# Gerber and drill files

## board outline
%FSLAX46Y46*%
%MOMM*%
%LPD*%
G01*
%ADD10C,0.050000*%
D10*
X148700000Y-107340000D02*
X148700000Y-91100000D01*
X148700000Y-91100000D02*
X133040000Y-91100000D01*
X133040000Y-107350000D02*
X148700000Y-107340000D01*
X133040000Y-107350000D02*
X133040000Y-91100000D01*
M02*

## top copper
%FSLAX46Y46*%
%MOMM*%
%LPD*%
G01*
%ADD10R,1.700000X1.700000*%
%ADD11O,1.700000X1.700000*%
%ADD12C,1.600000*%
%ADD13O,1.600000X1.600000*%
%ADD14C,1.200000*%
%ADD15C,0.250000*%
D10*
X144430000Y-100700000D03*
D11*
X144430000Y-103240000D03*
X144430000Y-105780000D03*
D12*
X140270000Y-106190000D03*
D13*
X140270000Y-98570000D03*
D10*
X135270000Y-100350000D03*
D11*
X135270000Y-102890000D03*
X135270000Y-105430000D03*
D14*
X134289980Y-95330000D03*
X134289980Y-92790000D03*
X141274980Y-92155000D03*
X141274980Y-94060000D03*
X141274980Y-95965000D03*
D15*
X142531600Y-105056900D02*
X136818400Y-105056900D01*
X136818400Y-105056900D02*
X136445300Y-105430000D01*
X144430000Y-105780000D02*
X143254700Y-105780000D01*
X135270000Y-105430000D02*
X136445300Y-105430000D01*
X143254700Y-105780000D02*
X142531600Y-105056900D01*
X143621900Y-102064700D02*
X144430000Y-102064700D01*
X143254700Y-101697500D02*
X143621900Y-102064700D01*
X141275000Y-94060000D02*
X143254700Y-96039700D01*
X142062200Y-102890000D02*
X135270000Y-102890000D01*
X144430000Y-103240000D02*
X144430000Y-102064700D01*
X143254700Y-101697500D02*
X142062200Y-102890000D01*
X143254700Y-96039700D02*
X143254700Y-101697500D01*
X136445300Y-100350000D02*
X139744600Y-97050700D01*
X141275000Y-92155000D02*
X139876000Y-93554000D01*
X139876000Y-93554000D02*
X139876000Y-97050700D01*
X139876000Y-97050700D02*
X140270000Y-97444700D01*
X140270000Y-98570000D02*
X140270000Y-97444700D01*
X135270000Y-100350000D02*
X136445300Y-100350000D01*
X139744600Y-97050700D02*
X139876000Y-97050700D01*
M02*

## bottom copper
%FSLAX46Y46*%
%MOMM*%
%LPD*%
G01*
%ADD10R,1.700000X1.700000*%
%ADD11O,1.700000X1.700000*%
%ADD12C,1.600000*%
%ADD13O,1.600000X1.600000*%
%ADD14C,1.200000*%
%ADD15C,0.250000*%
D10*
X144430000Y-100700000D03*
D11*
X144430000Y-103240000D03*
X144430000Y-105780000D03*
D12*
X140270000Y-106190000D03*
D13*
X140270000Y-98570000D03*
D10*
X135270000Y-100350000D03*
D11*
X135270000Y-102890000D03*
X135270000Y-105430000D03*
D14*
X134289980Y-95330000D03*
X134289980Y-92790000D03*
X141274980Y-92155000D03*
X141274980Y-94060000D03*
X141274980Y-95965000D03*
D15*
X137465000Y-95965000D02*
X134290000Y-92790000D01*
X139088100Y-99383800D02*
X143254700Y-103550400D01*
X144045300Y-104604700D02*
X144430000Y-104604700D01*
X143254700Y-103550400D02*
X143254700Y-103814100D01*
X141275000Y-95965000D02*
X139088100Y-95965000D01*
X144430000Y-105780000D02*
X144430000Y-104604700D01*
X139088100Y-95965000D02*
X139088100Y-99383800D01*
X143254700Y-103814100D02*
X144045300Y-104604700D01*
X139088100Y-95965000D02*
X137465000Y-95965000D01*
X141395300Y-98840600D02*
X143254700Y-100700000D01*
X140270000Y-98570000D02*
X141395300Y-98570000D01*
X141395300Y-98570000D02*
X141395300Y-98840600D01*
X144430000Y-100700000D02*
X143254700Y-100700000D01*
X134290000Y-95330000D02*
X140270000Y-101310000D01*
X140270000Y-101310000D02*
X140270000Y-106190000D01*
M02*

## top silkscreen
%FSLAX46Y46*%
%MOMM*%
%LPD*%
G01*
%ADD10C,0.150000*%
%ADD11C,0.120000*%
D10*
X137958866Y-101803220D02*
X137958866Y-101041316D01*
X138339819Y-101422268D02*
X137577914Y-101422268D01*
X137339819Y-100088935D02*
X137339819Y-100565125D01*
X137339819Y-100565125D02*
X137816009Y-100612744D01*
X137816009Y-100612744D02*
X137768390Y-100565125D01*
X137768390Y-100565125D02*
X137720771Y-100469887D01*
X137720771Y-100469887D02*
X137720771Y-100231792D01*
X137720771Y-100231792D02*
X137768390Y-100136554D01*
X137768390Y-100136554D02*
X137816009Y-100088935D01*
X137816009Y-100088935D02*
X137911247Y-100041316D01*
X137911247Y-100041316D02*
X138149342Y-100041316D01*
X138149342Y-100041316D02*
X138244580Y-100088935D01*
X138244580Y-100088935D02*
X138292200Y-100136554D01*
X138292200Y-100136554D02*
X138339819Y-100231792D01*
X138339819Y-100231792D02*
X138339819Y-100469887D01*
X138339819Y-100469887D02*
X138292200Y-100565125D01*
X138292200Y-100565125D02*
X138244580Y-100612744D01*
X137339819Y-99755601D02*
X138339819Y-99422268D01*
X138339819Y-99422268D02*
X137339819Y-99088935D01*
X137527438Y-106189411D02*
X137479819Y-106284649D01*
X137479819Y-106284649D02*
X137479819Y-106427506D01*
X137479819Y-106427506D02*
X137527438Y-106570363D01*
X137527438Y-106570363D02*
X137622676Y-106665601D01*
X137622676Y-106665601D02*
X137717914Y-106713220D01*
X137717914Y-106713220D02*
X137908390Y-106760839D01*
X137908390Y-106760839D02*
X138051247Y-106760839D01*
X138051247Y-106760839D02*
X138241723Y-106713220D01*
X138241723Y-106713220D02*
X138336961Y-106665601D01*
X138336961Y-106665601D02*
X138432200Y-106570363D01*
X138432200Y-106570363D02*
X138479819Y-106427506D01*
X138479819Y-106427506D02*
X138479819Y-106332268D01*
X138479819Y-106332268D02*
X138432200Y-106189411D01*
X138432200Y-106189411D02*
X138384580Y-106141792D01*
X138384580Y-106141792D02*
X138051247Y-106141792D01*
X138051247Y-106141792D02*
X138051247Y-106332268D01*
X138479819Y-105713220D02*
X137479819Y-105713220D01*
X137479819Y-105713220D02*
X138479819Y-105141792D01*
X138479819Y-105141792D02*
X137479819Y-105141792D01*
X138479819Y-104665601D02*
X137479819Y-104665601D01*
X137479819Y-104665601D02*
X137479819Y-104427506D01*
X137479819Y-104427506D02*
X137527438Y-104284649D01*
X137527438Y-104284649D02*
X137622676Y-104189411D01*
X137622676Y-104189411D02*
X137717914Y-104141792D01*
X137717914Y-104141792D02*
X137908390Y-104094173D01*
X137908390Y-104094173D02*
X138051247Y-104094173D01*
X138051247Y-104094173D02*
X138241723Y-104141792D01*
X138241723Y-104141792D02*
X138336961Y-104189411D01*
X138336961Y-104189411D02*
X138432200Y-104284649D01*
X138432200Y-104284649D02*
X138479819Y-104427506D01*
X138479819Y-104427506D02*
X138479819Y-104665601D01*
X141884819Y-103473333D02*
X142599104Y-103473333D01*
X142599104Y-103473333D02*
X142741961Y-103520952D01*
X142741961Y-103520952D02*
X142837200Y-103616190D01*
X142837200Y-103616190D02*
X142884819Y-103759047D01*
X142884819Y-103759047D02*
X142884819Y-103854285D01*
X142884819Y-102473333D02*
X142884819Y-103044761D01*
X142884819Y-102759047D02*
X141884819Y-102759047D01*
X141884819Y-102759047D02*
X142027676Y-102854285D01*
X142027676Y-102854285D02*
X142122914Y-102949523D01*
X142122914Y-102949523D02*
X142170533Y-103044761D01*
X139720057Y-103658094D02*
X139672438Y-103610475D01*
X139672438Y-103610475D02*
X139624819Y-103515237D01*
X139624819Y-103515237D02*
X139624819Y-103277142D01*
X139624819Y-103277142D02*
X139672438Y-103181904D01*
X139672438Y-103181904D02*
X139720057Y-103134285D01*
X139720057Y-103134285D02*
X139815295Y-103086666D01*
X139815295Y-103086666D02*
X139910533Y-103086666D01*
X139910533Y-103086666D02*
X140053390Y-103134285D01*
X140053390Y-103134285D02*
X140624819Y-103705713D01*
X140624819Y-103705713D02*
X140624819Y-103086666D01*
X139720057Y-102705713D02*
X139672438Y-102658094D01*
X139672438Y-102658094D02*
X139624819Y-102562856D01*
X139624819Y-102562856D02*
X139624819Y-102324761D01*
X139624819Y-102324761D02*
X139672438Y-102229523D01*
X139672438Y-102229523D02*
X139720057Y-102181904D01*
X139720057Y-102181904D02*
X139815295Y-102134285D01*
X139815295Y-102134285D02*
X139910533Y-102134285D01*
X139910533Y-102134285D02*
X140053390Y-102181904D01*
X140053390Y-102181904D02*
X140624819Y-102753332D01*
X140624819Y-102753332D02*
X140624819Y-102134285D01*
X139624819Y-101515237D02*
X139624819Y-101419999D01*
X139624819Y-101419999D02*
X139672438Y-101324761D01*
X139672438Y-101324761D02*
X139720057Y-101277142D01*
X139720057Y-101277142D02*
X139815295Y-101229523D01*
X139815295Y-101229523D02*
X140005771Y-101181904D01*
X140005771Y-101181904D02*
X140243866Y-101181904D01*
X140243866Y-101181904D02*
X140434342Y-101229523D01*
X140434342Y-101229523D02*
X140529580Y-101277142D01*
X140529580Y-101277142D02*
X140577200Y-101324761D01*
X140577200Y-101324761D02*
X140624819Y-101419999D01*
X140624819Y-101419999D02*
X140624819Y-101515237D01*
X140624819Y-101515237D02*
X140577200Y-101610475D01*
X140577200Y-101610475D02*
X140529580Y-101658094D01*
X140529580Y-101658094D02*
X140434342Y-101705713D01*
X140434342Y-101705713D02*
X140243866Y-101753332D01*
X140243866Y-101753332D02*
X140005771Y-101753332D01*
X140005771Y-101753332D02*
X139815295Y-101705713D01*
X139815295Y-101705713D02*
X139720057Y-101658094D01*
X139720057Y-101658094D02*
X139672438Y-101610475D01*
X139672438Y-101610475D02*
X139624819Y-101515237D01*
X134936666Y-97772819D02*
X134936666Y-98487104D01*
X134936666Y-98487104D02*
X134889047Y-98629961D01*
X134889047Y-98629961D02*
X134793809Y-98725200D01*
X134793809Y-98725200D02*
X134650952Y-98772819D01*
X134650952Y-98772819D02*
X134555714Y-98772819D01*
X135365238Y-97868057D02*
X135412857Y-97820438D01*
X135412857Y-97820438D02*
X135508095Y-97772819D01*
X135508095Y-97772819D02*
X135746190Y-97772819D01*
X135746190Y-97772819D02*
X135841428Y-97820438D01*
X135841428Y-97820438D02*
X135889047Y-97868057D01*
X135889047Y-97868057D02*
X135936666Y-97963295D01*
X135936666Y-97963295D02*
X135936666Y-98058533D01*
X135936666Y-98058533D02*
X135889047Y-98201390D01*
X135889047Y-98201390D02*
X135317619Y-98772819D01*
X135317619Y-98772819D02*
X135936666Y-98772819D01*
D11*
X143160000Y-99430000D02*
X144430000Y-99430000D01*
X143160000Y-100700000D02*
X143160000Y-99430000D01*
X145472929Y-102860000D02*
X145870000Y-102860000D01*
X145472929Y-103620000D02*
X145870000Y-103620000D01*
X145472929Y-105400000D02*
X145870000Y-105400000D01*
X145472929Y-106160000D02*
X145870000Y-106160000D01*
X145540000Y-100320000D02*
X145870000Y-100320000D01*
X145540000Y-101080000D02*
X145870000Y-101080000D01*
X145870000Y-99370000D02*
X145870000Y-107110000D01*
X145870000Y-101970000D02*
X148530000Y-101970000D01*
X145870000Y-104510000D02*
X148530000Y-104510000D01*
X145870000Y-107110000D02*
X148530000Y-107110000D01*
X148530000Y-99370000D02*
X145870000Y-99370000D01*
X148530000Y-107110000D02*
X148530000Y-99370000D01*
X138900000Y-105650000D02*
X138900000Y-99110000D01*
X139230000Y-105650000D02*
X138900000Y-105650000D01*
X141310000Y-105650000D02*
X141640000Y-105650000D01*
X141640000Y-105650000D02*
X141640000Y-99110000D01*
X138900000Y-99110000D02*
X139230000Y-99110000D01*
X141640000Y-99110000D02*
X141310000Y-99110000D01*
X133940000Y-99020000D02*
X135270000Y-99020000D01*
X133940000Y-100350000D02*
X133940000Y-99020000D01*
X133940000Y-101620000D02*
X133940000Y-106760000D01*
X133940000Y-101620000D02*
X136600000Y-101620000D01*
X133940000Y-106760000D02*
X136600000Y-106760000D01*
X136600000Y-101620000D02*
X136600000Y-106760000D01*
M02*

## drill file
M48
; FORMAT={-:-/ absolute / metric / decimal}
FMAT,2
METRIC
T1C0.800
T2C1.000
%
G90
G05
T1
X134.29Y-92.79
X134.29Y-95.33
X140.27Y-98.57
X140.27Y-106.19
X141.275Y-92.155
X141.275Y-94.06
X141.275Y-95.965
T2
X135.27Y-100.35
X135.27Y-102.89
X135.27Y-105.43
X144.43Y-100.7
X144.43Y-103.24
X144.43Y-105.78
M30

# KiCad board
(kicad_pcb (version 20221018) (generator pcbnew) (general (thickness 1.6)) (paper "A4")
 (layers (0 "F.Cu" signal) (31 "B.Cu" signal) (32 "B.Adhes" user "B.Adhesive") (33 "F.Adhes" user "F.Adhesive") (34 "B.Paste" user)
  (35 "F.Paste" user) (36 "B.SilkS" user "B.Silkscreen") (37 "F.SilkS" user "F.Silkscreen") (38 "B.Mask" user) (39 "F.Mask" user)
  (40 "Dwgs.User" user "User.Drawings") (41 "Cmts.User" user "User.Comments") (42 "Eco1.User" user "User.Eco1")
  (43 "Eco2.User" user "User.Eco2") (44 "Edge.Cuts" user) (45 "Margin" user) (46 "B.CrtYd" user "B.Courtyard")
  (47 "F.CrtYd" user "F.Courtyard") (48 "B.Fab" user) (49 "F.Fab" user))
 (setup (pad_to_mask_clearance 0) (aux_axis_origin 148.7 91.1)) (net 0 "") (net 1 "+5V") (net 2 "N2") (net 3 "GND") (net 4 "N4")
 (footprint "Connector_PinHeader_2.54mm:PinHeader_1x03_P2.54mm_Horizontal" (layer "F.Cu") (at 144.43 100.7)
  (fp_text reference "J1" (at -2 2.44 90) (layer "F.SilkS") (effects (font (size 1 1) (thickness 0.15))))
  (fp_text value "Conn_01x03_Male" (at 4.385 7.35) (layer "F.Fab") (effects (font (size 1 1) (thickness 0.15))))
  (fp_line (start -1.27 -1.27) (end 0 -1.27) (stroke (width 0.12) (type solid)) (layer "F.SilkS"))
  (fp_line (start -1.27 0) (end -1.27 -1.27) (stroke (width 0.12) (type solid)) (layer "F.SilkS"))
  (fp_line (start 1.042929 2.16) (end 1.44 2.16) (stroke (width 0.12) (type solid)) (layer "F.SilkS"))
  (fp_line (start 1.042929 2.92) (end 1.44 2.92) (stroke (width 0.12) (type solid)) (layer "F.SilkS"))
  (fp_line (start 1.042929 4.7) (end 1.44 4.7) (stroke (width 0.12) (type solid)) (layer "F.SilkS"))
  (fp_line (start 1.042929 5.46) (end 1.44 5.46) (stroke (width 0.12) (type solid)) (layer "F.SilkS"))
  (fp_line (start 1.11 -0.38) (end 1.44 -0.38) (stroke (width 0.12) (type solid)) (layer "F.SilkS"))
  (fp_line (start 1.11 0.38) (end 1.44 0.38) (stroke (width 0.12) (type solid)) (layer "F.SilkS"))
  (fp_line (start 1.44 -1.33) (end 1.44 6.41) (stroke (width 0.12) (type solid)) (layer "F.SilkS"))
  (fp_line (start 1.44 1.27) (end 4.1 1.27) (stroke (width 0.12) (type solid)) (layer "F.SilkS"))
  (fp_line (start 1.44 3.81) (end 4.1 3.81) (stroke (width 0.12) (type solid)) (layer "F.SilkS"))
  (fp_line (start 1.44 6.41) (end 4.1 6.41) (stroke (width 0.12) (type solid)) (layer "F.SilkS"))
  (fp_line (start 4.1 -1.33) (end 1.44 -1.33) (stroke (width 0.12) (type solid)) (layer "F.SilkS"))
  (fp_line (start 4.1 6.41) (end 4.1 -1.33) (stroke (width 0.12) (type solid)) (layer "F.SilkS"))
  (pad "1" thru_hole rect (at 0 0) (size 1.7 1.7) (drill 1) (layers "*.Cu" "*.Mask") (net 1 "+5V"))
  (pad "2" thru_hole oval (at 0 2.54) (size 1.7 1.7) (drill 1) (layers "*.Cu" "*.Mask") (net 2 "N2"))
  (pad "3" thru_hole oval (at 0 5.08) (size 1.7 1.7) (drill 1) (layers "*.Cu" "*.Mask") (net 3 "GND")))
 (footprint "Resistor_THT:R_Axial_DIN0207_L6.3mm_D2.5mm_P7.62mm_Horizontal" (layer "F.Cu") (at 140.27 106.19 90)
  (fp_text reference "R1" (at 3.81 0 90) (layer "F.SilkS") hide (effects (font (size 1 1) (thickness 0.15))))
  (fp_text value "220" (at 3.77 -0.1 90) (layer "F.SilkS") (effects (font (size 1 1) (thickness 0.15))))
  (fp_line (start 0.54 -1.37) (end 7.08 -1.37) (stroke (width 0.12) (type solid)) (layer "F.SilkS"))
  (fp_line (start 0.54 -1.04) (end 0.54 -1.37) (stroke (width 0.12) (type solid)) (layer "F.SilkS"))
  (fp_line (start 0.54 1.04) (end 0.54 1.37) (stroke (width 0.12) (type solid)) (layer "F.SilkS"))
  (fp_line (start 0.54 1.37) (end 7.08 1.37) (stroke (width 0.12) (type solid)) (layer "F.SilkS"))
  (fp_line (start 7.08 -1.37) (end 7.08 -1.04) (stroke (width 0.12) (type solid)) (layer "F.SilkS"))
  (fp_line (start 7.08 1.37) (end 7.08 1.04) (stroke (width 0.12) (type solid)) (layer "F.SilkS"))
  (pad "1" thru_hole circle (at 0 0 90) (size 1.6 1.6) (drill 0.8) (layers "*.Cu" "*.Mask") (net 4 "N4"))
  (pad "2" thru_hole oval (at 7.62 0 90) (size 1.6 1.6) (drill 0.8) (layers "*.Cu" "*.Mask") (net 1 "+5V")))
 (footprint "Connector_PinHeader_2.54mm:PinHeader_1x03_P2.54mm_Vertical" (layer "F.Cu") (at 135.27 100.35)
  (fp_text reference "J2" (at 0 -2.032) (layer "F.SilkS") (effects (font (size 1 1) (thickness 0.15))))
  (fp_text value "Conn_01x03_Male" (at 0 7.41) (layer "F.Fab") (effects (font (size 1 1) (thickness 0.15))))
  (fp_line (start -1.33 -1.33) (end 0 -1.33) (stroke (width 0.12) (type solid)) (layer "F.SilkS"))
  (fp_line (start -1.33 0) (end -1.33 -1.33) (stroke (width 0.12) (type solid)) (layer "F.SilkS"))
  (fp_line (start -1.33 1.27) (end -1.33 6.41) (stroke (width 0.12) (type solid)) (layer "F.SilkS"))
  (fp_line (start -1.33 1.27) (end 1.33 1.27) (stroke (width 0.12) (type solid)) (layer "F.SilkS"))
  (fp_line (start -1.33 6.41) (end 1.33 6.41) (stroke (width 0.12) (type solid)) (layer "F.SilkS"))
  (fp_line (start 1.33 1.27) (end 1.33 6.41) (stroke (width 0.12) (type solid)) (layer "F.SilkS"))
  (pad "1" thru_hole rect (at 0 0) (size 1.7 1.7) (drill 1) (layers "*.Cu" "*.Mask") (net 1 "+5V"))
  (pad "2" thru_hole oval (at 0 2.54) (size 1.7 1.7) (drill 1) (layers "*.Cu" "*.Mask") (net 2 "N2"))
  (pad "3" thru_hole oval (at 0 5.08) (size 1.7 1.7) (drill 1) (layers "*.Cu" "*.Mask") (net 3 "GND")))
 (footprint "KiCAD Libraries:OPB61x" (layer "B.Cu") (at 134.2898 95.3298)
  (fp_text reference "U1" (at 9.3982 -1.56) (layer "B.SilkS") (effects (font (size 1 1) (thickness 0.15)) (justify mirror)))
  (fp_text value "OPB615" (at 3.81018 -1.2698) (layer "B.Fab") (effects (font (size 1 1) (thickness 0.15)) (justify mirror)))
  (pad "1" thru_hole circle (at 0.00018 0.0002) (size 1.2 1.2) (drill 0.8) (layers "*.Cu" "*.Mask") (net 4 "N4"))
  (pad "2" thru_hole circle (at 0.00018 -2.5398) (size 1.2 1.2) (drill 0.8) (layers "*.Cu" "*.Mask") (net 3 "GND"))
  (pad "3" thru_hole circle (at 6.98518 -3.1748) (size 1.2 1.2) (drill 0.8) (layers "*.Cu" "*.Mask") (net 1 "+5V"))
  (pad "4" thru_hole circle (at 6.98518 -1.2698) (size 1.2 1.2) (drill 0.8) (layers "*.Cu" "*.Mask") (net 2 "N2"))
  (pad "5" thru_hole circle (at 6.98518 0.6352) (size 1.2 1.2) (drill 0.8) (layers "*.Cu" "*.Mask") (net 3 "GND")))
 (gr_line (start 148.7 107.34) (end 148.7 91.1) (stroke (width 0.05) (type solid)) (layer "Edge.Cuts"))
 (gr_line (start 148.7 91.1) (end 133.04 91.1) (stroke (width 0.05) (type solid)) (layer "Edge.Cuts"))
 (gr_line (start 133.04 107.35) (end 148.7 107.34) (stroke (width 0.05) (type solid)) (layer "Edge.Cuts"))
 (gr_line (start 133.04 107.35) (end 133.04 91.1) (stroke (width 0.05) (type solid)) (layer "Edge.Cuts"))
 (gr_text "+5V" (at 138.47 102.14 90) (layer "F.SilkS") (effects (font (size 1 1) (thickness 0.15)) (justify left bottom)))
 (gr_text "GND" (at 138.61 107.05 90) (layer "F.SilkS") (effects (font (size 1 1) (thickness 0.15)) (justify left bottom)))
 (segment (start 142.5316 105.0569) (end 136.8184 105.0569) (width 0.25) (layer "F.Cu") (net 3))
 (segment (start 136.8184 105.0569) (end 136.4453 105.43) (width 0.25) (layer "F.Cu") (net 3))
 (segment (start 144.43 105.78) (end 143.2547 105.78) (width 0.25) (layer "F.Cu") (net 3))
 (segment (start 135.27 105.43) (end 136.4453 105.43) (width 0.25) (layer "F.Cu") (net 3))
 (segment (start 143.2547 105.78) (end 142.5316 105.0569) (width 0.25) (layer "F.Cu") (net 3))
 (segment (start 137.465 95.965) (end 134.29 92.79) (width 0.25) (layer "B.Cu") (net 3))
 (segment (start 139.0881 99.3838) (end 143.2547 103.5504) (width 0.25) (layer "B.Cu") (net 3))
 (segment (start 144.0453 104.6047) (end 144.43 104.6047) (width 0.25) (layer "B.Cu") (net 3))
 (segment (start 143.2547 103.5504) (end 143.2547 103.8141) (width 0.25) (layer "B.Cu") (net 3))
 (segment (start 141.275 95.965) (end 139.0881 95.965) (width 0.25) (layer "B.Cu") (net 3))
 (segment (start 144.43 105.78) (end 144.43 104.6047) (width 0.25) (layer "B.Cu") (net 3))
 (segment (start 139.0881 95.965) (end 139.0881 99.3838) (width 0.25) (layer "B.Cu") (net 3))
 (segment (start 143.2547 103.8141) (end 144.0453 104.6047) (width 0.25) (layer "B.Cu") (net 3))
 (segment (start 139.0881 95.965) (end 137.465 95.965) (width 0.25) (layer "B.Cu") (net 3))
 (segment (start 143.6219 102.0647) (end 144.43 102.0647) (width 0.25) (layer "F.Cu") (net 2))
 (segment (start 143.2547 101.6975) (end 143.6219 102.0647) (width 0.25) (layer "F.Cu") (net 2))
 (segment (start 141.275 94.06) (end 143.2547 96.0397) (width 0.25) (layer "F.Cu") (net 2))
 (segment (start 142.0622 102.89) (end 135.27 102.89) (width 0.25) (layer "F.Cu") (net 2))
 (segment (start 144.43 103.24) (end 144.43 102.0647) (width 0.25) (layer "F.Cu") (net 2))
 (segment (start 143.2547 101.6975) (end 142.0622 102.89) (width 0.25) (layer "F.Cu") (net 2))
 (segment (start 143.2547 96.0397) (end 143.2547 101.6975) (width 0.25) (layer "F.Cu") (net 2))
 (segment (start 136.4453 100.35) (end 139.7446 97.0507) (width 0.25) (layer "F.Cu") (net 1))
 (segment (start 141.275 92.155) (end 139.876 93.554) (width 0.25) (layer "F.Cu") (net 1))
 (segment (start 139.876 93.554) (end 139.876 97.0507) (width 0.25) (layer "F.Cu") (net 1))
 (segment (start 139.876 97.0507) (end 140.27 97.4447) (width 0.25) (layer "F.Cu") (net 1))
 (segment (start 140.27 98.57) (end 140.27 97.4447) (width 0.25) (layer "F.Cu") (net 1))
 (segment (start 135.27 100.35) (end 136.4453 100.35) (width 0.25) (layer "F.Cu") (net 1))
 (segment (start 139.7446 97.0507) (end 139.876 97.0507) (width 0.25) (layer "F.Cu") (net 1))
 (segment (start 141.3953 98.8406) (end 143.2547 100.7) (width 0.25) (layer "B.Cu") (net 1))
 (segment (start 140.27 98.57) (end 141.3953 98.57) (width 0.25) (layer "B.Cu") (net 1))
 (segment (start 141.3953 98.57) (end 141.3953 98.8406) (width 0.25) (layer "B.Cu") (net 1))
 (segment (start 144.43 100.7) (end 143.2547 100.7) (width 0.25) (layer "B.Cu") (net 1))
 (segment (start 134.29 95.33) (end 140.27 101.31) (width 0.25) (layer "B.Cu") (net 4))
 (segment (start 140.27 101.31) (end 140.27 106.19) (width 0.25) (layer "B.Cu") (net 4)))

